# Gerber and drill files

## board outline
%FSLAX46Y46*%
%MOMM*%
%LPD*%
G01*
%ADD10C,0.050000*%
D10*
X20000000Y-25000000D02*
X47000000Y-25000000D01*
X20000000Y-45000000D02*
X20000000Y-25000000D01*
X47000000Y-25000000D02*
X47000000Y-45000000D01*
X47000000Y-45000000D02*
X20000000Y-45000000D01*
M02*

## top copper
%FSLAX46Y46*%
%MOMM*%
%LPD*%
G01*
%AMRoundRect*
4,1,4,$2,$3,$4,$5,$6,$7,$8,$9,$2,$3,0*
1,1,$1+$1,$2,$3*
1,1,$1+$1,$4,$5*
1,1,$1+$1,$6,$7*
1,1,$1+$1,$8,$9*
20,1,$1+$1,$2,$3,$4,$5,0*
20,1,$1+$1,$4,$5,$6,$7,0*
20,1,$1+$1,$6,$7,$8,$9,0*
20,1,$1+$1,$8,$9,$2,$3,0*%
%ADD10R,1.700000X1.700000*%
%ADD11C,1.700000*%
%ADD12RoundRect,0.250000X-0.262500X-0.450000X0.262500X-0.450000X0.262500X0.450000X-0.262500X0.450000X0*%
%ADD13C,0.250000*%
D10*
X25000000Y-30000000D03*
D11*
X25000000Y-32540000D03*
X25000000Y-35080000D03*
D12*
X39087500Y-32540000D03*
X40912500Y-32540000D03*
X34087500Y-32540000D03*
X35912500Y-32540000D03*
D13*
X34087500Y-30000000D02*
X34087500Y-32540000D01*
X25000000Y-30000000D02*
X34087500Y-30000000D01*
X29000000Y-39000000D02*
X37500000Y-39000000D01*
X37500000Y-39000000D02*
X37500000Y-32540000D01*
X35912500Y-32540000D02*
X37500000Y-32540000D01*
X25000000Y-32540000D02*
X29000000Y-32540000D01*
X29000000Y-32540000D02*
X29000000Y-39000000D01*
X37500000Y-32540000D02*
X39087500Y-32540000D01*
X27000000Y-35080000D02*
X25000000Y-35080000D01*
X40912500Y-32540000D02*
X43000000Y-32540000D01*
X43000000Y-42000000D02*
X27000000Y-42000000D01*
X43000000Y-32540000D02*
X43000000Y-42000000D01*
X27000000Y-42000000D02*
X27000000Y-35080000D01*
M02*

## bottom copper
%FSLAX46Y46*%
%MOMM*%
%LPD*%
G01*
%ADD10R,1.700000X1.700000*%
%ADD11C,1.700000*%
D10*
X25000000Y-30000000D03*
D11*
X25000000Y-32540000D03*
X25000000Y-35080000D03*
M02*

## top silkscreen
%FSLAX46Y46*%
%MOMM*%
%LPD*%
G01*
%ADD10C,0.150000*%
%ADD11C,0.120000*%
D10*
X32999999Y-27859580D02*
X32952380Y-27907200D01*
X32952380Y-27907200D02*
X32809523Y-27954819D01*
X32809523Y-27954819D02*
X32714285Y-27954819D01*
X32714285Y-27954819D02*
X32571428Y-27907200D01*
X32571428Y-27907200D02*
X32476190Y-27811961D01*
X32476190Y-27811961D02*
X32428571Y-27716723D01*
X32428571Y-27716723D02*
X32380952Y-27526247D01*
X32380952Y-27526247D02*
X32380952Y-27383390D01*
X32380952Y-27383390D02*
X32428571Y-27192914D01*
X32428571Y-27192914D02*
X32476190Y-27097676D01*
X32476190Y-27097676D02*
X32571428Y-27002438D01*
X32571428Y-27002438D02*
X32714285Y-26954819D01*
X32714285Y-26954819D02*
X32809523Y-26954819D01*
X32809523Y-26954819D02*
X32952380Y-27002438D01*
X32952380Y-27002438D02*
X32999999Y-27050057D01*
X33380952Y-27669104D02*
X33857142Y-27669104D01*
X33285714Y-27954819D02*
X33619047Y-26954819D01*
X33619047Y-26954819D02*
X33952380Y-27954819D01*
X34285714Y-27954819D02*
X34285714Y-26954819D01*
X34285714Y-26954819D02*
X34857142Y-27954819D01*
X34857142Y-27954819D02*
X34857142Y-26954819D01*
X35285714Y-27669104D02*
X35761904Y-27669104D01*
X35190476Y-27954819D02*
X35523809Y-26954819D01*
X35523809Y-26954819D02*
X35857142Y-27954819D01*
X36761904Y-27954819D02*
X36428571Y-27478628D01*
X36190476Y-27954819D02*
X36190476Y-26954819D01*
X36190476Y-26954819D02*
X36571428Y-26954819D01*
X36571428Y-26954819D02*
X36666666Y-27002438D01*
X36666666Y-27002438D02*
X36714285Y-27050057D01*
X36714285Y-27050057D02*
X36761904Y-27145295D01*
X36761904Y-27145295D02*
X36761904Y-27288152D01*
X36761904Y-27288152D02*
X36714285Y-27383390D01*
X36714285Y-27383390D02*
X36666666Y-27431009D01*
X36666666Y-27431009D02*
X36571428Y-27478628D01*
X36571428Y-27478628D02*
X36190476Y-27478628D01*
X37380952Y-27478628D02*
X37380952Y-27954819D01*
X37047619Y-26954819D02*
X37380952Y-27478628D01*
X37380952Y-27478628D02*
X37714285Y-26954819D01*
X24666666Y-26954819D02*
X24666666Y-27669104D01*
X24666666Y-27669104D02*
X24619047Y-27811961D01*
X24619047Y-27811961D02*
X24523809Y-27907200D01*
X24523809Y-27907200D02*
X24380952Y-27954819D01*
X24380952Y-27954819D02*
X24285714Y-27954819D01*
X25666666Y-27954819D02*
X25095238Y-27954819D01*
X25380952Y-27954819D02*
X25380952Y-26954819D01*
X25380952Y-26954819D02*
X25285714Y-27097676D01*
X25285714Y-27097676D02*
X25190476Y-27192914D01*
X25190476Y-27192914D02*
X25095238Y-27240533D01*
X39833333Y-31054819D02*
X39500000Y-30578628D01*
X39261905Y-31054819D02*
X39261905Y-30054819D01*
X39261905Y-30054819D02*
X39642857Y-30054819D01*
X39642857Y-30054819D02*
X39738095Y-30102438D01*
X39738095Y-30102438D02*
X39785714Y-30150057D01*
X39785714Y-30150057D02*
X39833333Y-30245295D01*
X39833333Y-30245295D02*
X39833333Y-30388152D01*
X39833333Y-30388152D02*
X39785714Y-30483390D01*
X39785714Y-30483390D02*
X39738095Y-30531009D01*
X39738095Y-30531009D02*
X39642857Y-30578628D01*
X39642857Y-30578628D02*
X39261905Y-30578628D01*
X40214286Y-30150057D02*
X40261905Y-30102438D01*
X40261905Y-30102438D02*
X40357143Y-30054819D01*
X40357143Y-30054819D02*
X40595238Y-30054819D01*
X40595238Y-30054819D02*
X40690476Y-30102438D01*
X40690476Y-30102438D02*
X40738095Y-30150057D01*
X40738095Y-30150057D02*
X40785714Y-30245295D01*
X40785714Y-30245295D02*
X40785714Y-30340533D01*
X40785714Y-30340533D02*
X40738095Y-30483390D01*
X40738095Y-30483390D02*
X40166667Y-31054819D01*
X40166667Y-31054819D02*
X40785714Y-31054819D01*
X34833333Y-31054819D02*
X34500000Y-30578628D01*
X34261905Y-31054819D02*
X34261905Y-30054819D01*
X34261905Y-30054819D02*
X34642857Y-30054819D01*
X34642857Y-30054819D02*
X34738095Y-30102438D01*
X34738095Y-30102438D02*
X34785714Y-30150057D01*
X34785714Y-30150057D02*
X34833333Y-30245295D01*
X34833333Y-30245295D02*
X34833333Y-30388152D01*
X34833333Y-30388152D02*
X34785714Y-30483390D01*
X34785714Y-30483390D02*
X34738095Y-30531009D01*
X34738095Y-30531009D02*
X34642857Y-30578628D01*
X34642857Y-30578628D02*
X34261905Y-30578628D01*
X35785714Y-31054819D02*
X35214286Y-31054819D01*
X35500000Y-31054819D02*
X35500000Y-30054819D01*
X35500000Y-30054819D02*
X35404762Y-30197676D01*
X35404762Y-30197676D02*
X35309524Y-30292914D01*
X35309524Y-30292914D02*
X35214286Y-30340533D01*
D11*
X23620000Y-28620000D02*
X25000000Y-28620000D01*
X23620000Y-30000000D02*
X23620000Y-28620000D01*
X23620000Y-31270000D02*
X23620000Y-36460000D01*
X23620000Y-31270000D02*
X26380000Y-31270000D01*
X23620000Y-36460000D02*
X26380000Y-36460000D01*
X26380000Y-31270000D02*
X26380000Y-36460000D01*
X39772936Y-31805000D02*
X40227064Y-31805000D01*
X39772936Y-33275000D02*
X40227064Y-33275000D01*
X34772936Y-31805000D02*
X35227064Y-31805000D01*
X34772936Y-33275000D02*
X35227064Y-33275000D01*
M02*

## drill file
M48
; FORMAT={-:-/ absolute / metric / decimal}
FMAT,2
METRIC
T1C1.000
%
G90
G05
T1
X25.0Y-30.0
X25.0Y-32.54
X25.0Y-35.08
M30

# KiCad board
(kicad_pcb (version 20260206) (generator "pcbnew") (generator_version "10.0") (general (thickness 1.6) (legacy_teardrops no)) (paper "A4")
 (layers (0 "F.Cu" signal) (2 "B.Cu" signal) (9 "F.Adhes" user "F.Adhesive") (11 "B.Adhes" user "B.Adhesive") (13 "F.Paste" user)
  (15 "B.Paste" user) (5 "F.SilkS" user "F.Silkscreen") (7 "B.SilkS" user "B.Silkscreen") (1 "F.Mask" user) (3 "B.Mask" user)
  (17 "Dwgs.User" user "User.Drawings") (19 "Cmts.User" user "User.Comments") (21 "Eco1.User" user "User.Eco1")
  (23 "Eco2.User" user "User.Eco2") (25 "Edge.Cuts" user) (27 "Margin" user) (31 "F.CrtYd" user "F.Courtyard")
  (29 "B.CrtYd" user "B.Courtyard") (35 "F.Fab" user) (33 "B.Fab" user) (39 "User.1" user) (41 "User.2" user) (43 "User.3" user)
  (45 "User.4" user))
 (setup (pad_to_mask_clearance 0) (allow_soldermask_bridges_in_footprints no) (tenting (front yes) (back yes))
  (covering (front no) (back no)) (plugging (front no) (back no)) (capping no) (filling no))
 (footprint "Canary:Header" (layer "F.Cu") (at 25 30)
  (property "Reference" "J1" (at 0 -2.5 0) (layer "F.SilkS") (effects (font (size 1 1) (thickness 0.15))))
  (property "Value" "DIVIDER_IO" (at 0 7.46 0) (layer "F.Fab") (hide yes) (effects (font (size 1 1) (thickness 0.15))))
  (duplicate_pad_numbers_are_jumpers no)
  (fp_line (start -1.38 -1.38) (end 0 -1.38) (stroke (width 0.12) (type solid)) (layer "F.SilkS"))
  (fp_line (start -1.38 0) (end -1.38 -1.38) (stroke (width 0.12) (type solid)) (layer "F.SilkS"))
  (fp_line (start -1.38 1.27) (end -1.38 6.46) (stroke (width 0.12) (type solid)) (layer "F.SilkS"))
  (fp_line (start -1.38 1.27) (end 1.38 1.27) (stroke (width 0.12) (type solid)) (layer "F.SilkS"))
  (fp_line (start -1.38 6.46) (end 1.38 6.46) (stroke (width 0.12) (type solid)) (layer "F.SilkS"))
  (fp_line (start 1.38 1.27) (end 1.38 6.46) (stroke (width 0.12) (type solid)) (layer "F.SilkS"))
  (pad "1" thru_hole rect (at 0 0) (size 1.7 1.7) (drill 1) (layers "*.Cu" "*.Mask") (remove_unused_layers no) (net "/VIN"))
  (pad "2" thru_hole circle (at 0 2.54) (size 1.7 1.7) (drill 1) (layers "*.Cu" "*.Mask") (remove_unused_layers no) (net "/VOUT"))
  (pad "3" thru_hole circle (at 0 5.08) (size 1.7 1.7) (drill 1) (layers "*.Cu" "*.Mask") (remove_unused_layers no) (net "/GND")))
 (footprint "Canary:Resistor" (layer "F.Cu") (at 40 32.54)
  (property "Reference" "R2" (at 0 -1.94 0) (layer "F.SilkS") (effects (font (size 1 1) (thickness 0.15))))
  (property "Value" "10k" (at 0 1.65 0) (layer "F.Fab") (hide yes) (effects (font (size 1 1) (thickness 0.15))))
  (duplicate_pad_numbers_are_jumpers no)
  (fp_line (start -0.227064 -0.735) (end 0.227064 -0.735) (stroke (width 0.12) (type solid)) (layer "F.SilkS"))
  (fp_line (start -0.227064 0.735) (end 0.227064 0.735) (stroke (width 0.12) (type solid)) (layer "F.SilkS"))
  (pad "1" smd roundrect (at -0.9125 0) (size 1.025 1.4) (layers "F.Cu" "F.Mask" "F.Paste") (roundrect_rratio 0.243902) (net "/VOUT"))
  (pad "2" smd roundrect (at 0.9125 0) (size 1.025 1.4) (layers "F.Cu" "F.Mask" "F.Paste") (roundrect_rratio 0.243902) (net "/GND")))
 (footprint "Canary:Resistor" (layer "F.Cu") (at 35 32.54)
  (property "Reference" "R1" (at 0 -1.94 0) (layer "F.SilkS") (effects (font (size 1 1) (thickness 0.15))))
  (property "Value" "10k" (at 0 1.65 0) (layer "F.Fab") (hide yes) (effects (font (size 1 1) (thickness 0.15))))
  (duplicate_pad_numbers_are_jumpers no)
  (fp_line (start -0.227064 -0.735) (end 0.227064 -0.735) (stroke (width 0.12) (type solid)) (layer "F.SilkS"))
  (fp_line (start -0.227064 0.735) (end 0.227064 0.735) (stroke (width 0.12) (type solid)) (layer "F.SilkS"))
  (pad "1" smd roundrect (at -0.9125 0) (size 1.025 1.4) (layers "F.Cu" "F.Mask" "F.Paste") (roundrect_rratio 0.243902) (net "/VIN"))
  (pad "2" smd roundrect (at 0.9125 0) (size 1.025 1.4) (layers "F.Cu" "F.Mask" "F.Paste") (roundrect_rratio 0.243902) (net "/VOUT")))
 (gr_line (start 20 25) (end 47 25) (stroke (width 0.05) (type default)) (layer "Edge.Cuts"))
 (gr_line (start 20 45) (end 20 25) (stroke (width 0.05) (type default)) (layer "Edge.Cuts"))
 (gr_line (start 47 25) (end 47 45) (stroke (width 0.05) (type default)) (layer "Edge.Cuts"))
 (gr_line (start 47 45) (end 20 45) (stroke (width 0.05) (type default)) (layer "Edge.Cuts"))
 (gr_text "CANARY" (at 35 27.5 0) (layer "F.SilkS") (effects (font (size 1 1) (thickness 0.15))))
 (segment (start 34.0875 30) (end 34.0875 32.54) (width 0.25) (layer "F.Cu") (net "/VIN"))
 (segment (start 25 30) (end 34.0875 30) (width 0.25) (layer "F.Cu") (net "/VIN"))
 (segment (start 29 39) (end 37.5 39) (width 0.25) (layer "F.Cu") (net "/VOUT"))
 (segment (start 37.5 39) (end 37.5 32.54) (width 0.25) (layer "F.Cu") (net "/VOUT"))
 (segment (start 35.9125 32.54) (end 37.5 32.54) (width 0.25) (layer "F.Cu") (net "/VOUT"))
 (segment (start 25 32.54) (end 29 32.54) (width 0.25) (layer "F.Cu") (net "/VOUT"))
 (segment (start 29 32.54) (end 29 39) (width 0.25) (layer "F.Cu") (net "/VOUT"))
 (segment (start 37.5 32.54) (end 39.0875 32.54) (width 0.25) (layer "F.Cu") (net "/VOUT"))
 (segment (start 27 35.08) (end 25 35.08) (width 0.25) (layer "F.Cu") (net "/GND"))
 (segment (start 40.9125 32.54) (end 43 32.54) (width 0.25) (layer "F.Cu") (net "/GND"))
 (segment (start 43 42) (end 27 42) (width 0.25) (layer "F.Cu") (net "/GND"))
 (segment (start 43 32.54) (end 43 42) (width 0.25) (layer "F.Cu") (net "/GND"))
 (segment (start 27 42) (end 27 35.08) (width 0.25) (layer "F.Cu") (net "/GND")))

